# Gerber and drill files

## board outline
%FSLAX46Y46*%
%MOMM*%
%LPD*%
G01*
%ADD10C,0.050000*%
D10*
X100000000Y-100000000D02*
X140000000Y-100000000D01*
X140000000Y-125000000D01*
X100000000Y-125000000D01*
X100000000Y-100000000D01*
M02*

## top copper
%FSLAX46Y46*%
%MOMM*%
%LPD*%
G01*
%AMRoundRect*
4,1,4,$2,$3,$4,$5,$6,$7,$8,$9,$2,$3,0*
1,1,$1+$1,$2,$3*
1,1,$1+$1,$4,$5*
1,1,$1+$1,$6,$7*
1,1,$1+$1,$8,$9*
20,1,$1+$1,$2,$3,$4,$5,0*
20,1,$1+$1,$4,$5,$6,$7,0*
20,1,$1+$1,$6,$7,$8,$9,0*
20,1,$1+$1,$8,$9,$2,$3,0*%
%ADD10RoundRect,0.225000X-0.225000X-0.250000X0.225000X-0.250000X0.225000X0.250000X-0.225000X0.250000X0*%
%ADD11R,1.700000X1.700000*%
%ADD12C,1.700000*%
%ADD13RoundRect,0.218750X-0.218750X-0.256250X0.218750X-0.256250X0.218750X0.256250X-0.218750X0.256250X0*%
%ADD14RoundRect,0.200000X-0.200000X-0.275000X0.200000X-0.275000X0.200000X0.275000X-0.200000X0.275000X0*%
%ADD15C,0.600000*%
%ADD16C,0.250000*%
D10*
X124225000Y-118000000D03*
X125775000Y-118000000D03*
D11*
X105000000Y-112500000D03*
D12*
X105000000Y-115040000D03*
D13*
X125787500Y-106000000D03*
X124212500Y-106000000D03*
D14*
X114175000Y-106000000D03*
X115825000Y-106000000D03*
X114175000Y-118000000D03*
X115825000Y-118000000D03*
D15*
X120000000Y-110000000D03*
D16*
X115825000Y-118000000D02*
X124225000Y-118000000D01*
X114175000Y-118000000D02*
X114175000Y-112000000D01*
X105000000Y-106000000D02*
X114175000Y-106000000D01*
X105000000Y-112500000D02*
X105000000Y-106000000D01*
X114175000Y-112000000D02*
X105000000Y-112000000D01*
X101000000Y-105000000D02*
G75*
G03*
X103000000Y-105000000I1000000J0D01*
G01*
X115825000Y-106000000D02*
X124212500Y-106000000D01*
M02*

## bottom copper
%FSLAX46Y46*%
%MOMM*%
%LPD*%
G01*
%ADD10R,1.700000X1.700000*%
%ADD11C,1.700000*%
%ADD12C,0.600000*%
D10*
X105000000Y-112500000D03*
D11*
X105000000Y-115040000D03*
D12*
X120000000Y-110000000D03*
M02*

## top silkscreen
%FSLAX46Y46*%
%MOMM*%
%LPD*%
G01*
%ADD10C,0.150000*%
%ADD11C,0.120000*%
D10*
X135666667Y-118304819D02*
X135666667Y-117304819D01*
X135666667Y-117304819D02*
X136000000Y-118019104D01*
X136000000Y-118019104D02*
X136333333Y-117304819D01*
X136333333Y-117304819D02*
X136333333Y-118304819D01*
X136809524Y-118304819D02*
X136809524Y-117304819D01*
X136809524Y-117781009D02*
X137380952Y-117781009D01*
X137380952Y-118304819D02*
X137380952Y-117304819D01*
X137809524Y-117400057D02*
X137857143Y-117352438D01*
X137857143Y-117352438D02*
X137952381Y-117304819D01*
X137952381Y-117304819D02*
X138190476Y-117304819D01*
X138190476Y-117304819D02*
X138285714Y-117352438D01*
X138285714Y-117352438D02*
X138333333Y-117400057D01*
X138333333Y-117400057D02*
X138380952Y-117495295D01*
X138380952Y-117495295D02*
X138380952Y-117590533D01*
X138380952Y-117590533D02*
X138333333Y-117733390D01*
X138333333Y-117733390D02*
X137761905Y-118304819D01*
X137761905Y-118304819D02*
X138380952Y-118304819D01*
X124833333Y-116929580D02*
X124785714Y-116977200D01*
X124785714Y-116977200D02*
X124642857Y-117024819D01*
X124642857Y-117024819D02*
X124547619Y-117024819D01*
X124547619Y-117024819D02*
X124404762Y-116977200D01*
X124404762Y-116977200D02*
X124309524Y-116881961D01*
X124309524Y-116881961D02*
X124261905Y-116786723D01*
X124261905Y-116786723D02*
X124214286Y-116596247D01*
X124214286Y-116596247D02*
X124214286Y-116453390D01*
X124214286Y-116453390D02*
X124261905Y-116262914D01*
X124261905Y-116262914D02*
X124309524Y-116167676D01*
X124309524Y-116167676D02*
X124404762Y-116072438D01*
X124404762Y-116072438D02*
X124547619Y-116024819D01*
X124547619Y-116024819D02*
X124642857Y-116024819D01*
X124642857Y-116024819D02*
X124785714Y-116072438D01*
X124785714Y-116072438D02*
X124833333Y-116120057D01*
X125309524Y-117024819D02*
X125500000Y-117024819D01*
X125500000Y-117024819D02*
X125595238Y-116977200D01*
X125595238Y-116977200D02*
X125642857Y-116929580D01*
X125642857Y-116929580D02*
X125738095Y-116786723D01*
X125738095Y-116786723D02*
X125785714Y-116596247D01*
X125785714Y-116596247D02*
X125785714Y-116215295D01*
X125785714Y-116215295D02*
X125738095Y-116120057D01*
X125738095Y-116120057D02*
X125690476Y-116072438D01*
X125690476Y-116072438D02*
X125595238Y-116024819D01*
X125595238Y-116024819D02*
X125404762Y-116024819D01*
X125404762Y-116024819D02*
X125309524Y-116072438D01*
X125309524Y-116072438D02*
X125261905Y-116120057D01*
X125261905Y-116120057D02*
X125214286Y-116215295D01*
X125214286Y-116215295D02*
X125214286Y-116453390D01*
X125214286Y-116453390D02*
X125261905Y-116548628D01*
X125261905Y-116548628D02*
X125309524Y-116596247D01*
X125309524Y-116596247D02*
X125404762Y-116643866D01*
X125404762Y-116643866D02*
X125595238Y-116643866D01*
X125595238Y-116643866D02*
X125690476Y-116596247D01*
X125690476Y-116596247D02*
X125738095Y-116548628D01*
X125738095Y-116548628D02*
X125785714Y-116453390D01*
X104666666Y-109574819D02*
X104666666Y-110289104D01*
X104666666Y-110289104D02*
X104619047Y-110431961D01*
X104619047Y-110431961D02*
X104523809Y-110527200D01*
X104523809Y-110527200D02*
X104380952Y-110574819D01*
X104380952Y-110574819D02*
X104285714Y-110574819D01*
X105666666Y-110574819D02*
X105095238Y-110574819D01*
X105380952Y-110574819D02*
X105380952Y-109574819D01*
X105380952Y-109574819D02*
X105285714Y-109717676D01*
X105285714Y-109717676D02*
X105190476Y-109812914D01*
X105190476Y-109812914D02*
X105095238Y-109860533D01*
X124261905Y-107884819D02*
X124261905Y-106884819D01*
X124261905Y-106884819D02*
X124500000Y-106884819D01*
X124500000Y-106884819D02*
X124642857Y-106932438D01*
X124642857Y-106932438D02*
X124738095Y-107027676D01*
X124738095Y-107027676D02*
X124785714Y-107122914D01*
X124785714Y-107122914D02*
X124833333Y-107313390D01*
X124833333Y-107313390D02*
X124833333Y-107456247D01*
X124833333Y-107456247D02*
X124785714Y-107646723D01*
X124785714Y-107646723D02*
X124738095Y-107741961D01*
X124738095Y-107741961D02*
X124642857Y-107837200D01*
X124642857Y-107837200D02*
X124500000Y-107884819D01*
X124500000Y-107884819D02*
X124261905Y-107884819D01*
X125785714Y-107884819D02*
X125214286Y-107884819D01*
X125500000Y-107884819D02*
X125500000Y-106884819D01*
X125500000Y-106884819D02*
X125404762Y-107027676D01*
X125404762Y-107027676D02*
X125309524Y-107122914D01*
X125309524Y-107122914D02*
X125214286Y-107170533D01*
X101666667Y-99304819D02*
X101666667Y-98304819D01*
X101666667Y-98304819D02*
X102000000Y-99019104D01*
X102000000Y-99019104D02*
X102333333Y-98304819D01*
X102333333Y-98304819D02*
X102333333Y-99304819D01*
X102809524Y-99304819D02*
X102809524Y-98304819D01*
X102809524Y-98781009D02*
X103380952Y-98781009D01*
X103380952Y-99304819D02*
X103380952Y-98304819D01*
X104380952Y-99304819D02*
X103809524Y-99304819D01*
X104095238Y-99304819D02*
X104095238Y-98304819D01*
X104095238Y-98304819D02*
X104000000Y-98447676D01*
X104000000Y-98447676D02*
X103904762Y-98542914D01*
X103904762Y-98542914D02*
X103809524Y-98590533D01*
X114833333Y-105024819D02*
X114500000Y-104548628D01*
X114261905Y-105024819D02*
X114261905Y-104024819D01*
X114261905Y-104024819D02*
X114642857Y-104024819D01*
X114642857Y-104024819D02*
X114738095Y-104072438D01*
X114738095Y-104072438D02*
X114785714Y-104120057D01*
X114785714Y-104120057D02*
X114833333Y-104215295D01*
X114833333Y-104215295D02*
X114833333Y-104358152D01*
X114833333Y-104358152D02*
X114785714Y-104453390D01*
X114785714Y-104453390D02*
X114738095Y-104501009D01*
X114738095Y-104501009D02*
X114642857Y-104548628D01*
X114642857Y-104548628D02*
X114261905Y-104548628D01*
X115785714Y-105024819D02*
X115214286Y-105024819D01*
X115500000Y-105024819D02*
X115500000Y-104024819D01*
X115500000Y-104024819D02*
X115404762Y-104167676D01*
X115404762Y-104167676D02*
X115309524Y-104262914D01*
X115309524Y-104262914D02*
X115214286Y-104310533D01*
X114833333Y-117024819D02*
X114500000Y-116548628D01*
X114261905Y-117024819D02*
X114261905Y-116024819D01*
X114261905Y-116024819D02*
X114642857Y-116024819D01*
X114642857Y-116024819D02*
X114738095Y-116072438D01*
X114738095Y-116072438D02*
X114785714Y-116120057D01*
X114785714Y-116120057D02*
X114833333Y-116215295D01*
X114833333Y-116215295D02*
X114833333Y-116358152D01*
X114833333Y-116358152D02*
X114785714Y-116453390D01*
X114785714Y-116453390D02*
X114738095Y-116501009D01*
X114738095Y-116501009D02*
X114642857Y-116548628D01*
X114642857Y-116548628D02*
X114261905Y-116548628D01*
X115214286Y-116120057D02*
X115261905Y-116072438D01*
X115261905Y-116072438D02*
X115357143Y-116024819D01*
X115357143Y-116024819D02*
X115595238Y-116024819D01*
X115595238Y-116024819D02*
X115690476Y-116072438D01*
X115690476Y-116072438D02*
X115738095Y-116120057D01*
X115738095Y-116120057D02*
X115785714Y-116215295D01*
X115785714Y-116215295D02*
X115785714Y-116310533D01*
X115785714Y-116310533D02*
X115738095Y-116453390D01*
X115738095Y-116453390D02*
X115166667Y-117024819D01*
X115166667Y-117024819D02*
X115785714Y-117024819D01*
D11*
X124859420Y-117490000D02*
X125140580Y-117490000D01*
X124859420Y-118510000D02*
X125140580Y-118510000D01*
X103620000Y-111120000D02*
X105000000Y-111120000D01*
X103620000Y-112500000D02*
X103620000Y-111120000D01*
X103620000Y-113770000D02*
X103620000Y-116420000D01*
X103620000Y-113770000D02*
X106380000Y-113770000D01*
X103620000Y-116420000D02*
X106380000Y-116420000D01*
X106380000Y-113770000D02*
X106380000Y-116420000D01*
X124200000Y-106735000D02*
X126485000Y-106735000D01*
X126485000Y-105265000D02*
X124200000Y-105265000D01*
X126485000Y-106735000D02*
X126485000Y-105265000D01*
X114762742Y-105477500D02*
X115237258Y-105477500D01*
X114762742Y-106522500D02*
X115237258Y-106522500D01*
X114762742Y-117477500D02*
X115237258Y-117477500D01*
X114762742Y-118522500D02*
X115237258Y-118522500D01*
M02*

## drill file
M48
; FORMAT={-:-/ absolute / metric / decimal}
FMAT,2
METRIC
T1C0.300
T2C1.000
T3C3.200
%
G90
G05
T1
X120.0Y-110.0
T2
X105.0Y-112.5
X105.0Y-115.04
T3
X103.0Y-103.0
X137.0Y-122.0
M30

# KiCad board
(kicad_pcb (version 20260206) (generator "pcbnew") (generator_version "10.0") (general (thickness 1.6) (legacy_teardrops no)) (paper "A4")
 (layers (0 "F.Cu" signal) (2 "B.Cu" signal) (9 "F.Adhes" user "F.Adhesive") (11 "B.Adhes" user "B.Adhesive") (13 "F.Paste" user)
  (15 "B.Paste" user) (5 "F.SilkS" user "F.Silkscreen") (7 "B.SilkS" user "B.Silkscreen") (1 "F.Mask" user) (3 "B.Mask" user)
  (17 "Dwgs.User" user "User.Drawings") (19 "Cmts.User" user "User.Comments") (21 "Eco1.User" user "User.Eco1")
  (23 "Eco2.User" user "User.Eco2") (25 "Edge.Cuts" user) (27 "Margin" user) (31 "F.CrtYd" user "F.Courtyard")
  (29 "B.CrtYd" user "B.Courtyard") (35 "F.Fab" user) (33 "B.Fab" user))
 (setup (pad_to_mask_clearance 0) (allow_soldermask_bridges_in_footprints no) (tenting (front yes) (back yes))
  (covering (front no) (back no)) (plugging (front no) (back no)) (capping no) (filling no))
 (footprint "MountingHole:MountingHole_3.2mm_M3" (layer "F.Cu") (at 137 122)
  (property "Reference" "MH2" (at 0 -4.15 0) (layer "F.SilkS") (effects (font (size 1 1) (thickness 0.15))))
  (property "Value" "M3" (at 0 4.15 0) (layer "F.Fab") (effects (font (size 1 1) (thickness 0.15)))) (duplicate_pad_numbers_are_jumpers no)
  (pad "" np_thru_hole circle (at 0 0) (size 3.2 3.2) (drill 3.2) (layers "*.Cu" "*.Mask")))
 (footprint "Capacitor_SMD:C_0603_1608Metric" (layer "F.Cu") (at 125 118)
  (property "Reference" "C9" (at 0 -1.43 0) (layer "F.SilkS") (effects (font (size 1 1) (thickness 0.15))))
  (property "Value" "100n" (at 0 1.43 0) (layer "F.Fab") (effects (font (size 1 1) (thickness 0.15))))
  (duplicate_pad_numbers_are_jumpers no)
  (fp_line (start -0.14058 -0.51) (end 0.14058 -0.51) (stroke (width 0.12) (type solid)) (layer "F.SilkS"))
  (fp_line (start -0.14058 0.51) (end 0.14058 0.51) (stroke (width 0.12) (type solid)) (layer "F.SilkS"))
  (pad "1" smd roundrect (at -0.775 0) (size 0.9 0.95) (layers "F.Cu" "F.Mask" "F.Paste") (roundrect_rratio 0.25) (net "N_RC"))
  (pad "2" smd roundrect (at 0.775 0) (size 0.9 0.95) (layers "F.Cu" "F.Mask" "F.Paste") (roundrect_rratio 0.25) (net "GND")))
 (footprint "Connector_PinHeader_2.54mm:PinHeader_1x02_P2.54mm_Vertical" (layer "F.Cu") (at 105 112.5)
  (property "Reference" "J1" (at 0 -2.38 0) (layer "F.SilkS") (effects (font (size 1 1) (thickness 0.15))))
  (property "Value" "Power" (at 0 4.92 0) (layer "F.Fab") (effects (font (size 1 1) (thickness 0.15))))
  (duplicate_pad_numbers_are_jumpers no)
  (fp_line (start -1.38 -1.38) (end 0 -1.38) (stroke (width 0.12) (type solid)) (layer "F.SilkS"))
  (fp_line (start -1.38 0) (end -1.38 -1.38) (stroke (width 0.12) (type solid)) (layer "F.SilkS"))
  (fp_line (start -1.38 1.27) (end -1.38 3.92) (stroke (width 0.12) (type solid)) (layer "F.SilkS"))
  (fp_line (start -1.38 1.27) (end 1.38 1.27) (stroke (width 0.12) (type solid)) (layer "F.SilkS"))
  (fp_line (start -1.38 3.92) (end 1.38 3.92) (stroke (width 0.12) (type solid)) (layer "F.SilkS"))
  (fp_line (start 1.38 1.27) (end 1.38 3.92) (stroke (width 0.12) (type solid)) (layer "F.SilkS"))
  (pad "1" thru_hole rect (at 0 0) (size 1.7 1.7) (drill 1) (layers "*.Cu" "*.Mask") (remove_unused_layers no) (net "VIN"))
  (pad "2" thru_hole circle (at 0 2.54) (size 1.7 1.7) (drill 1) (layers "*.Cu" "*.Mask") (remove_unused_layers no) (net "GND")))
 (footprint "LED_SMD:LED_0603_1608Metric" (layer "F.Cu") (at 125 106 180)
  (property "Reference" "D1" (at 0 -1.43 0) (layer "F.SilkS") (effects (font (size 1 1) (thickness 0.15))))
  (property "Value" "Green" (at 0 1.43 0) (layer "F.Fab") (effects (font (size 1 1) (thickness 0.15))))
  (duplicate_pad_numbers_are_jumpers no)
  (fp_line (start 0.8 -0.735) (end -1.485 -0.735) (stroke (width 0.12) (type solid)) (layer "F.SilkS"))
  (fp_line (start -1.485 0.735) (end 0.8 0.735) (stroke (width 0.12) (type solid)) (layer "F.SilkS"))
  (fp_line (start -1.485 -0.735) (end -1.485 0.735) (stroke (width 0.12) (type solid)) (layer "F.SilkS"))
  (pad "1" smd roundrect (at -0.7875 0) (size 0.875 0.95) (layers "F.Cu" "F.Mask" "F.Paste") (roundrect_rratio 0.25) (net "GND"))
  (pad "2" smd roundrect (at 0.7875 0) (size 0.875 0.95) (layers "F.Cu" "F.Mask" "F.Paste") (roundrect_rratio 0.25) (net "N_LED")))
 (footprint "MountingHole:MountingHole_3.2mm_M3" (layer "F.Cu") (at 103 103)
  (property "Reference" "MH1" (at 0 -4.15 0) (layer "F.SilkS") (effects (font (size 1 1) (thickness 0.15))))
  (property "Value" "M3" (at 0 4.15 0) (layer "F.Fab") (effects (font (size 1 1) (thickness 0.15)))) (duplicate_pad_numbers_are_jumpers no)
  (pad "" np_thru_hole circle (at 0 0) (size 3.2 3.2) (drill 3.2) (layers "*.Cu" "*.Mask")))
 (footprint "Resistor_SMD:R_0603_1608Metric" (layer "F.Cu") (at 115 106)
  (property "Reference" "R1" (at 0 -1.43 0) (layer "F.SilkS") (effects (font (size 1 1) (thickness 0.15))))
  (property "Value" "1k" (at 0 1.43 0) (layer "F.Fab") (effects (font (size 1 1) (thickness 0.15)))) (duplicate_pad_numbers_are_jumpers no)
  (fp_line (start -0.237258 -0.5225) (end 0.237258 -0.5225) (stroke (width 0.12) (type solid)) (layer "F.SilkS"))
  (fp_line (start -0.237258 0.5225) (end 0.237258 0.5225) (stroke (width 0.12) (type solid)) (layer "F.SilkS"))
  (pad "1" smd roundrect (at -0.825 0) (size 0.8 0.95) (layers "F.Cu" "F.Mask" "F.Paste") (roundrect_rratio 0.25) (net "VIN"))
  (pad "2" smd roundrect (at 0.825 0) (size 0.8 0.95) (layers "F.Cu" "F.Mask" "F.Paste") (roundrect_rratio 0.25) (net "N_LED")))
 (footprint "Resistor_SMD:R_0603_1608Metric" (layer "F.Cu") (at 115 118)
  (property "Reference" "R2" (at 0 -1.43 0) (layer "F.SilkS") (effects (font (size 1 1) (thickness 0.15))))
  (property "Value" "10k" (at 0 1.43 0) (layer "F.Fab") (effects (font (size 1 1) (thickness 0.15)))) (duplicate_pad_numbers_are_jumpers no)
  (fp_line (start -0.237258 -0.5225) (end 0.237258 -0.5225) (stroke (width 0.12) (type solid)) (layer "F.SilkS"))
  (fp_line (start -0.237258 0.5225) (end 0.237258 0.5225) (stroke (width 0.12) (type solid)) (layer "F.SilkS"))
  (pad "1" smd roundrect (at -0.825 0) (size 0.8 0.95) (layers "F.Cu" "F.Mask" "F.Paste") (roundrect_rratio 0.25) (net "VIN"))
  (pad "2" smd roundrect (at 0.825 0) (size 0.8 0.95) (layers "F.Cu" "F.Mask" "F.Paste") (roundrect_rratio 0.25) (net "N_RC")))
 (gr_rect (start 100 100) (end 140 125) (stroke (width 0.05) (type default)) (fill no) (layer "Edge.Cuts"))
 (segment (start 115.825 118) (end 124.225 118) (width 0.25) (layer "F.Cu") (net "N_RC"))
 (segment (start 114.175 118) (end 114.175 112) (width 0.25) (layer "F.Cu") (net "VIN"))
 (segment (start 105 106) (end 114.175 106) (width 0.25) (layer "F.Cu") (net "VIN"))
 (segment (start 105 112.5) (end 105 106) (width 0.25) (layer "F.Cu") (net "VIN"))
 (segment (start 114.175 112) (end 105 112) (width 0.25) (layer "F.Cu") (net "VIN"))
 (via (at 120 110) (size 0.6) (drill 0.3) (layers "F.Cu" "B.Cu") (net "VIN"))
 (arc (start 101 105) (mid 102 106) (end 103 105) (width 0.25) (layer "F.Cu") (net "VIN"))
 (segment (start 115.825 106) (end 124.2125 106) (width 0.25) (layer "F.Cu") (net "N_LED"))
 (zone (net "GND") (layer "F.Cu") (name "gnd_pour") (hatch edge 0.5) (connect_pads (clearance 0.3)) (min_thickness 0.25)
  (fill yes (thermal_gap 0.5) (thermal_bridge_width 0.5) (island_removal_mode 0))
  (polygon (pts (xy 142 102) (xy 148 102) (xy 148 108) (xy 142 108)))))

